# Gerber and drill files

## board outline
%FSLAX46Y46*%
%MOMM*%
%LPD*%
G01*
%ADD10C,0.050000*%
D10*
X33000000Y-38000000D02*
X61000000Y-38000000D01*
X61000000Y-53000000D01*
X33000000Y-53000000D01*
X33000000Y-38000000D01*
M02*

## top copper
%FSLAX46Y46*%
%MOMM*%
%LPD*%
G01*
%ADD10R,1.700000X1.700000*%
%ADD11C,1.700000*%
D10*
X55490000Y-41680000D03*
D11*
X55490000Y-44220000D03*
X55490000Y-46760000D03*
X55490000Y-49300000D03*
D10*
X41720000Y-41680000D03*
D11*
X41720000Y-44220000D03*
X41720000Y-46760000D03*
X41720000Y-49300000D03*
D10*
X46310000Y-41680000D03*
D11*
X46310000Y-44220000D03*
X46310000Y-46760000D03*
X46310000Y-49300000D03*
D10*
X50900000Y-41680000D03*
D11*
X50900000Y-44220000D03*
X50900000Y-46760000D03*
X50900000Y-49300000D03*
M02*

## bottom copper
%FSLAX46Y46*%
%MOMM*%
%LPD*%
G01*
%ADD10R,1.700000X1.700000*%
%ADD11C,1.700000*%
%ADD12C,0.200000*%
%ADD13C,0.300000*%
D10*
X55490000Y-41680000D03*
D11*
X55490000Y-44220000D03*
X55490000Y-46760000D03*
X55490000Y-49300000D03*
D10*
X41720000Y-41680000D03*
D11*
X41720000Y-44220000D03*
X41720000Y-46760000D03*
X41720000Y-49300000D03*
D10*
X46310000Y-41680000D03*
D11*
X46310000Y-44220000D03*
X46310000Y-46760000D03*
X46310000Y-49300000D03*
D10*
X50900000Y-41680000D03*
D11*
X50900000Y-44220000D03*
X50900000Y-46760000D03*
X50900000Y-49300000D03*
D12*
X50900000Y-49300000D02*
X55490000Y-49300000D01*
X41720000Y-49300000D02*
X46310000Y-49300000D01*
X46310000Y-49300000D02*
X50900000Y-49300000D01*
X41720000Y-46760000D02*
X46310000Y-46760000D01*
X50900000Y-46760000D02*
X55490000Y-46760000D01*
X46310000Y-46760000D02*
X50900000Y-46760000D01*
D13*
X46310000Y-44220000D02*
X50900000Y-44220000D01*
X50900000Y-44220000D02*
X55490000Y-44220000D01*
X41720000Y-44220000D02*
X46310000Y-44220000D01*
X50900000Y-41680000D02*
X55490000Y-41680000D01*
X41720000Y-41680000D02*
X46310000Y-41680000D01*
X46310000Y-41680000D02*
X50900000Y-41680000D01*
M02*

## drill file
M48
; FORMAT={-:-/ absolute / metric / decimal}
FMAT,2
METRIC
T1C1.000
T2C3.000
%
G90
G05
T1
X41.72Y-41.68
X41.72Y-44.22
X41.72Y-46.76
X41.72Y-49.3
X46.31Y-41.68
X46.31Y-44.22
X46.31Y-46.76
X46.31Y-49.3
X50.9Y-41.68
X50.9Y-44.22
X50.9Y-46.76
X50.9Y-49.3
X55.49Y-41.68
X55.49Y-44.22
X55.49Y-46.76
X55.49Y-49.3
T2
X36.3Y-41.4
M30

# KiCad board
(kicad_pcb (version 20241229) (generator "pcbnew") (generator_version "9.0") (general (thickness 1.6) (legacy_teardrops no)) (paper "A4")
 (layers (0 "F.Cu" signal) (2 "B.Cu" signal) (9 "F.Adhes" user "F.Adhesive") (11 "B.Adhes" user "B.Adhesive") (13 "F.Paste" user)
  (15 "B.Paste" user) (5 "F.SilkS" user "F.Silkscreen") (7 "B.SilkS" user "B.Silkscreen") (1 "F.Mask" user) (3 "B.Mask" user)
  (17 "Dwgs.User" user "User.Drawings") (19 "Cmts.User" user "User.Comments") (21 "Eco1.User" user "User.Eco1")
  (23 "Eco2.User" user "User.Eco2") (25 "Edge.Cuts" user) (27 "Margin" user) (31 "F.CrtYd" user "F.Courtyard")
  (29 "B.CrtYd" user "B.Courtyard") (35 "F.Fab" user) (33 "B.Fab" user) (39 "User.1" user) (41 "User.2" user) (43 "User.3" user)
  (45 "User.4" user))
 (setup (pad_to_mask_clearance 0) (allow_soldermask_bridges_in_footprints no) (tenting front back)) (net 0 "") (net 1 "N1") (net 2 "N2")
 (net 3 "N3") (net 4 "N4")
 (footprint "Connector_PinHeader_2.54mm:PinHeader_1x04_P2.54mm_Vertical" (layer "F.Cu") (at 55.49 41.68)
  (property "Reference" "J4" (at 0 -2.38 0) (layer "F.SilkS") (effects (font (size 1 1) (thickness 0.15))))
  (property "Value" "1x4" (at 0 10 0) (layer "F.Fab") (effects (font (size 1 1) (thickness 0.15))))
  (pad "1" thru_hole rect (at 0 0) (size 1.7 1.7) (drill 1) (layers "*.Cu" "*.Mask") (remove_unused_layers no) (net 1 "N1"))
  (pad "2" thru_hole circle (at 0 2.54) (size 1.7 1.7) (drill 1) (layers "*.Cu" "*.Mask") (remove_unused_layers no) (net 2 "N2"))
  (pad "3" thru_hole circle (at 0 5.08) (size 1.7 1.7) (drill 1) (layers "*.Cu" "*.Mask") (remove_unused_layers no) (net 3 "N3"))
  (pad "4" thru_hole circle (at 0 7.62) (size 1.7 1.7) (drill 1) (layers "*.Cu" "*.Mask") (remove_unused_layers no) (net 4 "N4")))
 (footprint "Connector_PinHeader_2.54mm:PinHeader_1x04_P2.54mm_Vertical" (layer "F.Cu") (at 41.72 41.68)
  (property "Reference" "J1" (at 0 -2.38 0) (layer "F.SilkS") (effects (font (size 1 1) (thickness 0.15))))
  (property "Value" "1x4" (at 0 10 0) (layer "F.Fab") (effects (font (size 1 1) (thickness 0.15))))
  (pad "1" thru_hole rect (at 0 0) (size 1.7 1.7) (drill 1) (layers "*.Cu" "*.Mask") (remove_unused_layers no) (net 1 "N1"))
  (pad "2" thru_hole circle (at 0 2.54) (size 1.7 1.7) (drill 1) (layers "*.Cu" "*.Mask") (remove_unused_layers no) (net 2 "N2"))
  (pad "3" thru_hole circle (at 0 5.08) (size 1.7 1.7) (drill 1) (layers "*.Cu" "*.Mask") (remove_unused_layers no) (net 3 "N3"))
  (pad "4" thru_hole circle (at 0 7.62) (size 1.7 1.7) (drill 1) (layers "*.Cu" "*.Mask") (remove_unused_layers no) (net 4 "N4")))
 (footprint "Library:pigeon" (layer "F.Cu") (at 36.5 48.9)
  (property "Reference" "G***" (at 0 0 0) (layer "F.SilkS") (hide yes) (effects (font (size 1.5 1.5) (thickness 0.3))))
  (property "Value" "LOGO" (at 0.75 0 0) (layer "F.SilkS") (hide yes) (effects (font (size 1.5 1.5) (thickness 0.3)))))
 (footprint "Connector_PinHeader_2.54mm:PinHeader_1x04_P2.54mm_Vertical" (layer "F.Cu") (at 46.31 41.68)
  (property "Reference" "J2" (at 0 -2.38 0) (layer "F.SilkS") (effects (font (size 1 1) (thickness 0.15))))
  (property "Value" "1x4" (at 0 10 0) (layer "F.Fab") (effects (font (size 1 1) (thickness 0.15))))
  (pad "1" thru_hole rect (at 0 0) (size 1.7 1.7) (drill 1) (layers "*.Cu" "*.Mask") (remove_unused_layers no) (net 1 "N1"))
  (pad "2" thru_hole circle (at 0 2.54) (size 1.7 1.7) (drill 1) (layers "*.Cu" "*.Mask") (remove_unused_layers no) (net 2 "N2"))
  (pad "3" thru_hole circle (at 0 5.08) (size 1.7 1.7) (drill 1) (layers "*.Cu" "*.Mask") (remove_unused_layers no) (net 3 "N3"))
  (pad "4" thru_hole circle (at 0 7.62) (size 1.7 1.7) (drill 1) (layers "*.Cu" "*.Mask") (remove_unused_layers no) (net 4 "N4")))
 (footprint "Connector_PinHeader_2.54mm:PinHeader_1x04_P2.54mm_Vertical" (layer "F.Cu") (at 50.9 41.68)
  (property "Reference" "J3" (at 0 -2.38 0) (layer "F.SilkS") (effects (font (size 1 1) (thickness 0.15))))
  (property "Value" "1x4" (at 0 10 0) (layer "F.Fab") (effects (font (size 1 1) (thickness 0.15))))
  (pad "1" thru_hole rect (at 0 0) (size 1.7 1.7) (drill 1) (layers "*.Cu" "*.Mask") (remove_unused_layers no) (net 1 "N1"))
  (pad "2" thru_hole circle (at 0 2.54) (size 1.7 1.7) (drill 1) (layers "*.Cu" "*.Mask") (remove_unused_layers no) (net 2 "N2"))
  (pad "3" thru_hole circle (at 0 5.08) (size 1.7 1.7) (drill 1) (layers "*.Cu" "*.Mask") (remove_unused_layers no) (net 3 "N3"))
  (pad "4" thru_hole circle (at 0 7.62) (size 1.7 1.7) (drill 1) (layers "*.Cu" "*.Mask") (remove_unused_layers no) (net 4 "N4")))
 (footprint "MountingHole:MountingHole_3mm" (layer "F.Cu") (at 36.3 41.4)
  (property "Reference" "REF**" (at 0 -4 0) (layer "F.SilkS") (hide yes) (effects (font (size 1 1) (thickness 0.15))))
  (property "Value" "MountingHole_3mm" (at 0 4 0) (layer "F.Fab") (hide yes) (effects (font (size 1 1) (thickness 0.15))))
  (pad "" np_thru_hole circle (at 0 0) (size 3 3) (drill 3) (layers "*.Cu" "*.Mask")))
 (gr_rect (start 33 38) (end 61 53) (stroke (width 0.05) (type solid)) (fill no) (layer "Edge.Cuts"))
 (segment (start 50.9 49.3) (end 55.49 49.3) (width 0.2) (layer "B.Cu") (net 4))
 (segment (start 41.72 49.3) (end 46.31 49.3) (width 0.2) (layer "B.Cu") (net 4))
 (segment (start 46.31 49.3) (end 50.9 49.3) (width 0.2) (layer "B.Cu") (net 4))
 (segment (start 41.72 46.76) (end 46.31 46.76) (width 0.2) (layer "B.Cu") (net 3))
 (segment (start 50.9 46.76) (end 55.49 46.76) (width 0.2) (layer "B.Cu") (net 3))
 (segment (start 46.31 46.76) (end 50.9 46.76) (width 0.2) (layer "B.Cu") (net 3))
 (segment (start 46.31 44.22) (end 50.9 44.22) (width 0.3) (layer "B.Cu") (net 2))
 (segment (start 50.9 44.22) (end 55.49 44.22) (width 0.3) (layer "B.Cu") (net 2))
 (segment (start 41.72 44.22) (end 46.31 44.22) (width 0.3) (layer "B.Cu") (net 2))
 (segment (start 50.9 41.68) (end 55.49 41.68) (width 0.3) (layer "B.Cu") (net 1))
 (segment (start 41.72 41.68) (end 46.31 41.68) (width 0.3) (layer "B.Cu") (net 1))
 (segment (start 46.31 41.68) (end 50.9 41.68) (width 0.3) (layer "B.Cu") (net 1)))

